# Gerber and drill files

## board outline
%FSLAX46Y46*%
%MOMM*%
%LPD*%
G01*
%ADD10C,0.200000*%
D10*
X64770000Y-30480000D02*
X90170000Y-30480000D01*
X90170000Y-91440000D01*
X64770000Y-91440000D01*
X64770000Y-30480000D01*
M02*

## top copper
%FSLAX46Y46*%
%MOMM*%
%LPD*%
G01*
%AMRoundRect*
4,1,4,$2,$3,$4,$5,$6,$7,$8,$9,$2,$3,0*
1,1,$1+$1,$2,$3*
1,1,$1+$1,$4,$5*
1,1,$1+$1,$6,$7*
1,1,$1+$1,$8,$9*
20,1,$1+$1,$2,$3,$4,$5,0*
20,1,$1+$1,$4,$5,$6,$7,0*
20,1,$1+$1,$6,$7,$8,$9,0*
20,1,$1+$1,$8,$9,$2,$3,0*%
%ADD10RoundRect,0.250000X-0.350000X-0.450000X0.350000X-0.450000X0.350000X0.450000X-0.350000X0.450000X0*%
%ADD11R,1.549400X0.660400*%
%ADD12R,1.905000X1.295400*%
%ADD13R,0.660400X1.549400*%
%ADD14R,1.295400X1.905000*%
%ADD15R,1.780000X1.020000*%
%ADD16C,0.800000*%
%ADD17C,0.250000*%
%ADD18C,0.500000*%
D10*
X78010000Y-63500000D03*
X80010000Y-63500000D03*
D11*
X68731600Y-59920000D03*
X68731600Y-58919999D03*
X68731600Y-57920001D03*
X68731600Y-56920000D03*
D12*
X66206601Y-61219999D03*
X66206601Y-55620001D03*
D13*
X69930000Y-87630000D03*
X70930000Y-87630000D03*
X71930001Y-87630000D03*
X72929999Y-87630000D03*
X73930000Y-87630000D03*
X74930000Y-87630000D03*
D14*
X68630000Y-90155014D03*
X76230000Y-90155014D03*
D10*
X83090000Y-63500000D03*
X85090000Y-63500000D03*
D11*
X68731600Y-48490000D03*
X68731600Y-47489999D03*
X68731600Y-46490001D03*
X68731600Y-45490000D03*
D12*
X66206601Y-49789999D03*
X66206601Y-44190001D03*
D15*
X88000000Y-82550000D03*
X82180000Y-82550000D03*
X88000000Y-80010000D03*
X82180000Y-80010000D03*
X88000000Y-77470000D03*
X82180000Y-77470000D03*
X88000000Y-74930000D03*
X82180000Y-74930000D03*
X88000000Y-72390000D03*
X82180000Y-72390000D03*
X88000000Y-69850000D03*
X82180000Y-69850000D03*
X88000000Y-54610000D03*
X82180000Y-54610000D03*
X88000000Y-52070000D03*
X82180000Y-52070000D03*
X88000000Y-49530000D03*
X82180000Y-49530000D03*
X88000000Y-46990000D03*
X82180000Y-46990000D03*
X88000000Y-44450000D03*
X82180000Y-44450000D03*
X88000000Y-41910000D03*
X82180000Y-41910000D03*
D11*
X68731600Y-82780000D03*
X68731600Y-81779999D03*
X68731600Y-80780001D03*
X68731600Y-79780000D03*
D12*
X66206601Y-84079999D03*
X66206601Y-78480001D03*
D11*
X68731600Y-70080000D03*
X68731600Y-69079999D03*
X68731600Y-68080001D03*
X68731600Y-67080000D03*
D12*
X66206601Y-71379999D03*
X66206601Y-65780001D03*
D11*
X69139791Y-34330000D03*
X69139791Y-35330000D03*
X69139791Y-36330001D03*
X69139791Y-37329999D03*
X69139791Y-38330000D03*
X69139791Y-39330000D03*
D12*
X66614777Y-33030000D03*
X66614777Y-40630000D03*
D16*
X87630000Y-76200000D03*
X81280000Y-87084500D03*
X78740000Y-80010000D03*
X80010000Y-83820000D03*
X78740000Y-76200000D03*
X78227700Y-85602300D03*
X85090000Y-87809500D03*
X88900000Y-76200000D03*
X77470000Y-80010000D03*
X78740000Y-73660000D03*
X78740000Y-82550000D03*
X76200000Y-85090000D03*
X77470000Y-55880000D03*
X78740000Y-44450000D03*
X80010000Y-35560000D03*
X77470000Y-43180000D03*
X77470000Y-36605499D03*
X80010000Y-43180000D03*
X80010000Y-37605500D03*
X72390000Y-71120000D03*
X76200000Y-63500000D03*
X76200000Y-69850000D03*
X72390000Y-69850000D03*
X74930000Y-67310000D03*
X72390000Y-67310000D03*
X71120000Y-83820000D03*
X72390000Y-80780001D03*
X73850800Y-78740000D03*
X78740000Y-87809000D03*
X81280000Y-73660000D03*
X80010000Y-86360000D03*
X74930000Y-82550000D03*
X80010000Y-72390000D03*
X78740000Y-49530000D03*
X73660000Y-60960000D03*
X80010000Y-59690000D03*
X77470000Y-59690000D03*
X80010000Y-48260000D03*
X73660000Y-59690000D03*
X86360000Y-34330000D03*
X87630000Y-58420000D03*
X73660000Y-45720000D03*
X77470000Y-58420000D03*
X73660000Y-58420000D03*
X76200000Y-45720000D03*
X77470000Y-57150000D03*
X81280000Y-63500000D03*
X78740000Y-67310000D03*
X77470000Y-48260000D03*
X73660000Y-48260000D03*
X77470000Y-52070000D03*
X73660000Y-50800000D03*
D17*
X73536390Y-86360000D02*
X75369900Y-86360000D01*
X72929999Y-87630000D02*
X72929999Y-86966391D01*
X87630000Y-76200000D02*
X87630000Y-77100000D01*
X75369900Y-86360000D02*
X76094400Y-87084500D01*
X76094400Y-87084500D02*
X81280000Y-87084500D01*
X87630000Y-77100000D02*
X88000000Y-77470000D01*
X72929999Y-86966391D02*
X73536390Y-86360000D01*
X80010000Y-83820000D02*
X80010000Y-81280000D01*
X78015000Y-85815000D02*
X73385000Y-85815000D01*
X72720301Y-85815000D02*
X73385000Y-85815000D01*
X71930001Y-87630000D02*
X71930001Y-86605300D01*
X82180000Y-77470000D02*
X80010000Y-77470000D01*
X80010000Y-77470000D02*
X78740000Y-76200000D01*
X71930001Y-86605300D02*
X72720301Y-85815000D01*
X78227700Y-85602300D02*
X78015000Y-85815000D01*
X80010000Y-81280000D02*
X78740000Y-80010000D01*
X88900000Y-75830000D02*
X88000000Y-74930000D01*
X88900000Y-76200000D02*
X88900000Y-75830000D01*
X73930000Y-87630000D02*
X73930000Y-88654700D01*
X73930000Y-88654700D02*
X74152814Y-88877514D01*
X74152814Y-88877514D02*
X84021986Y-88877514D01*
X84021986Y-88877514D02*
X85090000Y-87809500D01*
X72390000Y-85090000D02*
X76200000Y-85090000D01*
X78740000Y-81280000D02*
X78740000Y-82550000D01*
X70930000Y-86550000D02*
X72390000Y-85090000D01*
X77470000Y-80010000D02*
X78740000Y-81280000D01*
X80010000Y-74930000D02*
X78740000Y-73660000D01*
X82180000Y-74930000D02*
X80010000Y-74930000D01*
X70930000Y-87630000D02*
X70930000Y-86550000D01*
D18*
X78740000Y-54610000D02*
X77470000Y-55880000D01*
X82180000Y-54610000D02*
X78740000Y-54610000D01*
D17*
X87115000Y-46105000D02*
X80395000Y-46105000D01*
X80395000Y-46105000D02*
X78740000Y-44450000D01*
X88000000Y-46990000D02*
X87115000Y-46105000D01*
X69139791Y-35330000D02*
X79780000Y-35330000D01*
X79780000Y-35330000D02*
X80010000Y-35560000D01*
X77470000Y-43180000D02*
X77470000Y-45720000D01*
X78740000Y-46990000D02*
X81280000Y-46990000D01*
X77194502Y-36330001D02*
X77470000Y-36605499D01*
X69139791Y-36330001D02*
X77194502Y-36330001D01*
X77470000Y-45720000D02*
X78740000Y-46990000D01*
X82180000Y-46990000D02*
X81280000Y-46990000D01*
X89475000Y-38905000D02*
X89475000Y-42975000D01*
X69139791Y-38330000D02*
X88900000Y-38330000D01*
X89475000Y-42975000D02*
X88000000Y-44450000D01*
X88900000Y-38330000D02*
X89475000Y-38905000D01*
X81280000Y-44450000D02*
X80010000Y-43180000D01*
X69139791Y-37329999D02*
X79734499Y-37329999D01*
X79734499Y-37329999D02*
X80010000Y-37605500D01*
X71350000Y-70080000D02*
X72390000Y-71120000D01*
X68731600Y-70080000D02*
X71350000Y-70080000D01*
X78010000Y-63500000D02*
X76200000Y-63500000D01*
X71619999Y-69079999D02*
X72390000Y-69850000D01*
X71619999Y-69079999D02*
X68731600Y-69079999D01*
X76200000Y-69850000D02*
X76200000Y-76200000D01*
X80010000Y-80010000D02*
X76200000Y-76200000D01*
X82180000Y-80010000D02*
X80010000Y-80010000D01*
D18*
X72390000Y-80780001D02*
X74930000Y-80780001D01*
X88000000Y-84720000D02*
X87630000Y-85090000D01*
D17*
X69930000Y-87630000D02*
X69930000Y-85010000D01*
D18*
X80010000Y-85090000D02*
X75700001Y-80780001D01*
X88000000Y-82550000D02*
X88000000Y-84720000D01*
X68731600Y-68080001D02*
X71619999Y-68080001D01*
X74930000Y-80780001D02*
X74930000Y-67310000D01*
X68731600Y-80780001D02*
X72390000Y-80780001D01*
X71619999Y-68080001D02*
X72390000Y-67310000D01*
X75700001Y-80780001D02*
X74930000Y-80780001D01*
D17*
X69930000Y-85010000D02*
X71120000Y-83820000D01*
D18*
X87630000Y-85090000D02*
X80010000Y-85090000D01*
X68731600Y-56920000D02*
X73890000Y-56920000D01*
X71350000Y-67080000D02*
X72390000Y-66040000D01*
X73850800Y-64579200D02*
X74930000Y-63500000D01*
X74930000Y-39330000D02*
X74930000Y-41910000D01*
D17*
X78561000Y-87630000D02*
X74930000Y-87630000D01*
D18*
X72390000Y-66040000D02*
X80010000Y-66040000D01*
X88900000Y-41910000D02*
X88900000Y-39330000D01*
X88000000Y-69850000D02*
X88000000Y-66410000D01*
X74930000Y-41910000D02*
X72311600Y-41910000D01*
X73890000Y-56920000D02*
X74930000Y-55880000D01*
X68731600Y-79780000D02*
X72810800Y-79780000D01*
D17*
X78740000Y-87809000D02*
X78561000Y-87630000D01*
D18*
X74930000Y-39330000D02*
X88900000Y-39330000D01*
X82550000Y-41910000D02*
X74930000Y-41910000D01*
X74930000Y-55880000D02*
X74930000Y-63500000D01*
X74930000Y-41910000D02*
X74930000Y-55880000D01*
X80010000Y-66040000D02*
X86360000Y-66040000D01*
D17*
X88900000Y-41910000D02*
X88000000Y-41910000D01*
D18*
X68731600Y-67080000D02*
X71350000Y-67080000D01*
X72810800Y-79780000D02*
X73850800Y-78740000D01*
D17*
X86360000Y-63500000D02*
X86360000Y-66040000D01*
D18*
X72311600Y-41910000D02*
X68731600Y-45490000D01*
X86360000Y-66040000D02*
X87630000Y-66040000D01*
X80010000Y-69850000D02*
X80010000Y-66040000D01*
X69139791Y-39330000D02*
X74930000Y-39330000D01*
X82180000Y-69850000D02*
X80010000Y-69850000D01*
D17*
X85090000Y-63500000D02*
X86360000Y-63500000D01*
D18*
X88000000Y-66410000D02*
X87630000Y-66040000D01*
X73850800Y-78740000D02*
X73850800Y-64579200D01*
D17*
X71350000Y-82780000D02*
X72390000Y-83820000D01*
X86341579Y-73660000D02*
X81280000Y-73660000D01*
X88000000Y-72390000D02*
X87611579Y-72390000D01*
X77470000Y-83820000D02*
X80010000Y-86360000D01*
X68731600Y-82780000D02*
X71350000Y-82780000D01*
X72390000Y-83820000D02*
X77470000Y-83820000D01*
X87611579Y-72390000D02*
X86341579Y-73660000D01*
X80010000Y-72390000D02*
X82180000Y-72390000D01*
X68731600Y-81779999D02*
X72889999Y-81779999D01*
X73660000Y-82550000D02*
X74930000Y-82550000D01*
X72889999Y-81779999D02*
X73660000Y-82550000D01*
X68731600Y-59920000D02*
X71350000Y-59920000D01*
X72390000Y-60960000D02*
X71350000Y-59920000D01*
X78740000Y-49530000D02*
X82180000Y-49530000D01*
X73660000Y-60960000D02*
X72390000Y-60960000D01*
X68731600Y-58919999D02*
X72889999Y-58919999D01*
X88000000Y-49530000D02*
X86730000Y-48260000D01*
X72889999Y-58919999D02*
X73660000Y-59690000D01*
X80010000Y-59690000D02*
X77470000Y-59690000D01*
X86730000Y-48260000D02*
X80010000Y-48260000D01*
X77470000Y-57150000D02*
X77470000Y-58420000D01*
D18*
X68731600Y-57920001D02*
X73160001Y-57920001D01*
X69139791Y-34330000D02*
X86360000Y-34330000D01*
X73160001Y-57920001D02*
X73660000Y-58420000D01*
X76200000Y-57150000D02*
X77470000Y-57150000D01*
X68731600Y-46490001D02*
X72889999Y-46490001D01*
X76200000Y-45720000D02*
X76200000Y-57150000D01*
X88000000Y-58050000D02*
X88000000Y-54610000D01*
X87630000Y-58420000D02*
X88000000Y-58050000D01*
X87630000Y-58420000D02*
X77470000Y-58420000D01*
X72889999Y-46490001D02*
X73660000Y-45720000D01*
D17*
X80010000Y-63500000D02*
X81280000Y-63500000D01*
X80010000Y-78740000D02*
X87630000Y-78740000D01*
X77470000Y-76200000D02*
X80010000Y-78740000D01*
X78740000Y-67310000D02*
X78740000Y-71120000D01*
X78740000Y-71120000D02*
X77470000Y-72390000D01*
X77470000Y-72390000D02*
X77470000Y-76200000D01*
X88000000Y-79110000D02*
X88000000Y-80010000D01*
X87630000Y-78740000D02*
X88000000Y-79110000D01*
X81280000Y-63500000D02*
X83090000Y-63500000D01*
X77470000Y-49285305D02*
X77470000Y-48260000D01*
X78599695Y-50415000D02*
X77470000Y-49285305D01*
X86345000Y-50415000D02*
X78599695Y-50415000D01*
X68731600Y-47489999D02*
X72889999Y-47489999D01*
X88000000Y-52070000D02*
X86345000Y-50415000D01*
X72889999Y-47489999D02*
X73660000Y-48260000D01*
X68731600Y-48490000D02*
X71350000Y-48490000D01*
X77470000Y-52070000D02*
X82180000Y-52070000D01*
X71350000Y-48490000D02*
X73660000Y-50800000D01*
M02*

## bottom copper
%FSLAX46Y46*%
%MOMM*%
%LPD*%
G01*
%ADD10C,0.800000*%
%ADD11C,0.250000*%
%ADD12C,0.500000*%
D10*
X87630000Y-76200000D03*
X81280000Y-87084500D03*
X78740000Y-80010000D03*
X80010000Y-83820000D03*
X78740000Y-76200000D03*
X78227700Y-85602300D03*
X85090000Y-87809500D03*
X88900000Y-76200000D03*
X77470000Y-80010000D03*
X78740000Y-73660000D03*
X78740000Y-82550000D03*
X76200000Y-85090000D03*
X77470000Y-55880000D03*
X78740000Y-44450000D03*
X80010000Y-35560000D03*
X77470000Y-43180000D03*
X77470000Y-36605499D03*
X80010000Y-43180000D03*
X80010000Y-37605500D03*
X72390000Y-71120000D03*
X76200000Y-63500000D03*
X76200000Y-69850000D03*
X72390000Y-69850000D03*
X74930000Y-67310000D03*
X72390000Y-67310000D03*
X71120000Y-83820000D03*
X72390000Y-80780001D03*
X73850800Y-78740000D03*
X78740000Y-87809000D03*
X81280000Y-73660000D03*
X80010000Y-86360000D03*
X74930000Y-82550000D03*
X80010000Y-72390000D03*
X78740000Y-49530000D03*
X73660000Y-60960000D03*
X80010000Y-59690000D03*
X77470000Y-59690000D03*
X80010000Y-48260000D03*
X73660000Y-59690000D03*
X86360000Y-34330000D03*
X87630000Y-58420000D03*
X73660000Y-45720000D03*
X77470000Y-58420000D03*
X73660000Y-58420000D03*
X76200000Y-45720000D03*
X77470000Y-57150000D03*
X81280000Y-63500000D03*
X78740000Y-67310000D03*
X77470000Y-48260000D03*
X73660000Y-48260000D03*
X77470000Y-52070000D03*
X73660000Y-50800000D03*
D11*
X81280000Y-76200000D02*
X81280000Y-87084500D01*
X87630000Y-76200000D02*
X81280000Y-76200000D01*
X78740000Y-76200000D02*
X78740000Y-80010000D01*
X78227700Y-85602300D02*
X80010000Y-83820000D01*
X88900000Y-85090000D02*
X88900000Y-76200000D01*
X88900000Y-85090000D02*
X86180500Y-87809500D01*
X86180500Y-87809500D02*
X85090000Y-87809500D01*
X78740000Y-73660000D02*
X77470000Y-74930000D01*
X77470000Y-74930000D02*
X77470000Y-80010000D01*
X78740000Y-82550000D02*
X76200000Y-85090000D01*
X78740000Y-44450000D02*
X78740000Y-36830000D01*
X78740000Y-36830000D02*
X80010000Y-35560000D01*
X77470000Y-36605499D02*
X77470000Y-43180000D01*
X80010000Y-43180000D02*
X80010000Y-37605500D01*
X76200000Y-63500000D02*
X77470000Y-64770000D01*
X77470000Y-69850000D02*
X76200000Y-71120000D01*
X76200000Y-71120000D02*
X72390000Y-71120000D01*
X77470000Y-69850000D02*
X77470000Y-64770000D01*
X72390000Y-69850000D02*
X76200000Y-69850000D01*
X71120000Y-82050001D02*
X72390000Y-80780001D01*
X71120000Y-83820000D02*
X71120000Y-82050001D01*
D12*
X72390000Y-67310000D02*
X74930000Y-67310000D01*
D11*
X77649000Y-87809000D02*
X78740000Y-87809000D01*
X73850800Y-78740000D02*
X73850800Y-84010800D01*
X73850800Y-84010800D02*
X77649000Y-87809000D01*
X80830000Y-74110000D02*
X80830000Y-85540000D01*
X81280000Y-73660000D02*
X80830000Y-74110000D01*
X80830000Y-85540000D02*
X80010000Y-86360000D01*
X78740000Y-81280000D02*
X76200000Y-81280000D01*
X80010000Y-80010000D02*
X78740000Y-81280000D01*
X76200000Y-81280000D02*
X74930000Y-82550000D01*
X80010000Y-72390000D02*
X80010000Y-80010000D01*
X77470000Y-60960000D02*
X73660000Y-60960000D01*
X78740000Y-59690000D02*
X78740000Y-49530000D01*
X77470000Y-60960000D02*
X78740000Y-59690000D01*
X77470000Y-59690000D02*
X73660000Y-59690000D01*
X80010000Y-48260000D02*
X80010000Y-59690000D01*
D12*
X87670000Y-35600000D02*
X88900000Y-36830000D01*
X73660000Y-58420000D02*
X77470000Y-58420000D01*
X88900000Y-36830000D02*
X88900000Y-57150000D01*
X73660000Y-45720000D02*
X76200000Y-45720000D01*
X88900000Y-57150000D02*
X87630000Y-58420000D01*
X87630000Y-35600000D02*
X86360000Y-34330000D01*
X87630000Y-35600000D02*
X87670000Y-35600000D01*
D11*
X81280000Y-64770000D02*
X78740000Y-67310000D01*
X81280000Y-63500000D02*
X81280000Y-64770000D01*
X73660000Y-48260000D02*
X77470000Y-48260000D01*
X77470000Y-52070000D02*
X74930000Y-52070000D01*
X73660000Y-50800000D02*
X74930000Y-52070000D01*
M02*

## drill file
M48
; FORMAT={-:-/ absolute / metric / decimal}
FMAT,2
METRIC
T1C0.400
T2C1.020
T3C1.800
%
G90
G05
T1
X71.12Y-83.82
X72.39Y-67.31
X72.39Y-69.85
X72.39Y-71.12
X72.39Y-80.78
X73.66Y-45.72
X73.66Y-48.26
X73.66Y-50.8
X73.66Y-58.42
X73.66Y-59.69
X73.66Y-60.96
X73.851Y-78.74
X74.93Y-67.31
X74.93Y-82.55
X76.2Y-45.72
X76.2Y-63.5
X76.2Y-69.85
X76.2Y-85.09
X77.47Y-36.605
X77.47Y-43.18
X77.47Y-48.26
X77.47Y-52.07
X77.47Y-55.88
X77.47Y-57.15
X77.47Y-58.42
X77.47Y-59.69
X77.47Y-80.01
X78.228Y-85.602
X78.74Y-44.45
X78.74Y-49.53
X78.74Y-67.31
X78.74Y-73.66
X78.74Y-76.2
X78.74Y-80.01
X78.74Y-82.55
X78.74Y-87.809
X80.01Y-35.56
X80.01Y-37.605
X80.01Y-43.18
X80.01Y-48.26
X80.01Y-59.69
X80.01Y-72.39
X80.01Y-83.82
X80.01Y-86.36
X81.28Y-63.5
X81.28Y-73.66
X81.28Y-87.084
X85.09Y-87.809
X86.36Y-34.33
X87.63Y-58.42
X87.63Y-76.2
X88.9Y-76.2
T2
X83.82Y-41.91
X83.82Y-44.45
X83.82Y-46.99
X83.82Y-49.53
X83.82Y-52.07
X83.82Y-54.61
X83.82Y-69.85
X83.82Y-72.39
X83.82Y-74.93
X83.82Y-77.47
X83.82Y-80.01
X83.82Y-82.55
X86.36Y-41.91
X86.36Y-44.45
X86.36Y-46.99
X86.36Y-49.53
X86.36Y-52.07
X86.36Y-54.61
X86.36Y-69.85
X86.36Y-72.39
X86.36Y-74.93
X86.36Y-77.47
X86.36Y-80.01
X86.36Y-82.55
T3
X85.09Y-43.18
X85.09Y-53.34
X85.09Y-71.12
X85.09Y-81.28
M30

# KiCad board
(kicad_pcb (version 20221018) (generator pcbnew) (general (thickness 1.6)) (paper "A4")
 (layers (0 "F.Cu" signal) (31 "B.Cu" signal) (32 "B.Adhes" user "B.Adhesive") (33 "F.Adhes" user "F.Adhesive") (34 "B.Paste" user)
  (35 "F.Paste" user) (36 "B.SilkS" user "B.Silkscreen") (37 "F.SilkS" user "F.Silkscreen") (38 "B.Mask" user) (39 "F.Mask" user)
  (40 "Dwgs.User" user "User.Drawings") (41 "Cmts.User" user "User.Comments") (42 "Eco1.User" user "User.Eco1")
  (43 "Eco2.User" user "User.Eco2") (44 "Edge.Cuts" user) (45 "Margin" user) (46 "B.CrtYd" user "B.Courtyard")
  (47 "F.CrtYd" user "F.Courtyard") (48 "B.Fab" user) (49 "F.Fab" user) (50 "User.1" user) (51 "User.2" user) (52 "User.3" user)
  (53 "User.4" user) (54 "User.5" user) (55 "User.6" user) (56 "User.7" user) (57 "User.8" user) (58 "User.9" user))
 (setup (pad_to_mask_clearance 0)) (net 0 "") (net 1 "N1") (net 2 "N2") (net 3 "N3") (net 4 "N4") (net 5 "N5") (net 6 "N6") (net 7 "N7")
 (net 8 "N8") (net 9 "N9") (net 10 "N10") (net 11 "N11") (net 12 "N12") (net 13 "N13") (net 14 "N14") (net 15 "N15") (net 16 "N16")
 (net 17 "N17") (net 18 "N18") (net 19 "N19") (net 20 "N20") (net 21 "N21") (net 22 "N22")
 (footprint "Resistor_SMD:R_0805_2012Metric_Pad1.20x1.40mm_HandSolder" (layer "F.Cu") (at 79.01 63.5)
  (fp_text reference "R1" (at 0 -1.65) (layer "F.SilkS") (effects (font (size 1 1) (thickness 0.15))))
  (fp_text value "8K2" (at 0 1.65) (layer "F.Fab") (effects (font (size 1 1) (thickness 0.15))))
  (pad "1" smd roundrect (at -1 0) (size 1.2 1.4) (layers "F.Cu" "F.Paste" "F.Mask") (roundrect_rratio 0.2083333333) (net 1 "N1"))
  (pad "2" smd roundrect (at 1 0) (size 1.2 1.4) (layers "F.Cu" "F.Paste" "F.Mask") (roundrect_rratio 0.2083333333) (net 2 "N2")))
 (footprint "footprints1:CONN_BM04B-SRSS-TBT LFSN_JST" (layer "F.Cu") (at 67.31 58.42 90)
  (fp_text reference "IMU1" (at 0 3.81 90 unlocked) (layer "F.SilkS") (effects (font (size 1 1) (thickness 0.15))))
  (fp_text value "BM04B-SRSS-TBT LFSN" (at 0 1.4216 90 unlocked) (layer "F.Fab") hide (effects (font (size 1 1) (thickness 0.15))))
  (pad "1" smd rect (at -1.5 1.4216 90) (size 0.6604 1.5494) (layers "F.Cu" "F.Paste" "F.Mask") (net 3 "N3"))
  (pad "2" smd rect (at -0.499999 1.4216 90) (size 0.6604 1.5494) (layers "F.Cu" "F.Paste" "F.Mask") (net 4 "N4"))
  (pad "3" smd rect (at 0.499999 1.4216 90) (size 0.6604 1.5494) (layers "F.Cu" "F.Paste" "F.Mask") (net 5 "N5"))
  (pad "4" smd rect (at 1.5 1.4216 90) (size 0.6604 1.5494) (layers "F.Cu" "F.Paste" "F.Mask") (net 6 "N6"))
  (pad "5" smd rect (at -2.799999 -1.103399 180) (size 1.905 1.2954) (layers "F.Cu" "F.Paste" "F.Mask"))
  (pad "6" smd rect (at 2.799999 -1.103399 180) (size 1.905 1.2954) (layers "F.Cu" "F.Paste" "F.Mask")))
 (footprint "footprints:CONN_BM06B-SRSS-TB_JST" (layer "F.Cu") (at 72.43 89.459791)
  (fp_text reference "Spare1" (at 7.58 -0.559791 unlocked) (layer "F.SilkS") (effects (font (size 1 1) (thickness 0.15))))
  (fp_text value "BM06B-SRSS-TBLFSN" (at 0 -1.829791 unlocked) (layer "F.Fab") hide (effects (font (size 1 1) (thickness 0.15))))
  (pad "1" smd rect (at -2.5 -1.829791) (size 0.6604 1.5494) (layers "F.Cu" "F.Paste" "F.Mask") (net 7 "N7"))
  (pad "2" smd rect (at -1.5 -1.829791) (size 0.6604 1.5494) (layers "F.Cu" "F.Paste" "F.Mask") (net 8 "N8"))
  (pad "3" smd rect (at -0.499999 -1.829791) (size 0.6604 1.5494) (layers "F.Cu" "F.Paste" "F.Mask") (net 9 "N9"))
  (pad "4" smd rect (at 0.499999 -1.829791) (size 0.6604 1.5494) (layers "F.Cu" "F.Paste" "F.Mask") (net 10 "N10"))
  (pad "5" smd rect (at 1.5 -1.829791) (size 0.6604 1.5494) (layers "F.Cu" "F.Paste" "F.Mask") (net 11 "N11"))
  (pad "6" smd rect (at 2.5 -1.829791) (size 0.6604 1.5494) (layers "F.Cu" "F.Paste" "F.Mask") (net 6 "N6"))
  (pad "7" smd rect (at -3.8 0.695223 90) (size 1.905 1.2954) (layers "F.Cu" "F.Paste" "F.Mask"))
  (pad "8" smd rect (at 3.8 0.695223 90) (size 1.905 1.2954) (layers "F.Cu" "F.Paste" "F.Mask")))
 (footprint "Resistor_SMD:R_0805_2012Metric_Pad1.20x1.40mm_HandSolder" (layer "F.Cu") (at 84.09 63.5)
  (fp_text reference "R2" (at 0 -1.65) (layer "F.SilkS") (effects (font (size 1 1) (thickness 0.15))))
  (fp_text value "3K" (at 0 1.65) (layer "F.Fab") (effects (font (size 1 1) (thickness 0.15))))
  (pad "1" smd roundrect (at -1 0) (size 1.2 1.4) (layers "F.Cu" "F.Paste" "F.Mask") (roundrect_rratio 0.2083333333) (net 2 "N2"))
  (pad "2" smd roundrect (at 1 0) (size 1.2 1.4) (layers "F.Cu" "F.Paste" "F.Mask") (roundrect_rratio 0.2083333333) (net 6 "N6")))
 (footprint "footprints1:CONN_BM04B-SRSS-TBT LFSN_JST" (layer "F.Cu") (at 67.31 46.99 90)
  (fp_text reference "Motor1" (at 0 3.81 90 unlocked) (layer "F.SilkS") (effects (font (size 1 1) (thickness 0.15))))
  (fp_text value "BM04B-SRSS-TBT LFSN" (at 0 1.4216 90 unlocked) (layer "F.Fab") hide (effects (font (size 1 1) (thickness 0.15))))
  (pad "1" smd rect (at -1.5 1.4216 90) (size 0.6604 1.5494) (layers "F.Cu" "F.Paste" "F.Mask") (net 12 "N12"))
  (pad "2" smd rect (at -0.499999 1.4216 90) (size 0.6604 1.5494) (layers "F.Cu" "F.Paste" "F.Mask") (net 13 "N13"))
  (pad "3" smd rect (at 0.499999 1.4216 90) (size 0.6604 1.5494) (layers "F.Cu" "F.Paste" "F.Mask") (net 5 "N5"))
  (pad "4" smd rect (at 1.5 1.4216 90) (size 0.6604 1.5494) (layers "F.Cu" "F.Paste" "F.Mask") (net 6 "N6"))
  (pad "5" smd rect (at -2.799999 -1.103399 180) (size 1.905 1.2954) (layers "F.Cu" "F.Paste" "F.Mask"))
  (pad "6" smd rect (at 2.799999 -1.103399 180) (size 1.905 1.2954) (layers "F.Cu" "F.Paste" "F.Mask")))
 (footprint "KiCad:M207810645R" (layer "F.Cu") (at 85.09 76.2 90)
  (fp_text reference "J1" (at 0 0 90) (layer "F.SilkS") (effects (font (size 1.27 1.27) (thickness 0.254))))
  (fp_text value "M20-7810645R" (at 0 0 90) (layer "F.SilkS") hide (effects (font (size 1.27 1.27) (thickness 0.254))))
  (pad "" np_thru_hole circle (at -6.35 -1.27 90) (size 1.02 1.02) (drill 1.02) (layers "*.Cu" "*.Mask"))
  (pad "" np_thru_hole circle (at -6.35 1.27 90) (size 1.02 1.02) (drill 1.02) (layers "*.Cu" "*.Mask"))
  (pad "" np_thru_hole circle (at -5.08 0 90) (size 1.8 1.8) (drill 1.8) (layers "*.Cu" "*.Mask"))
  (pad "" np_thru_hole circle (at -3.81 -1.27 90) (size 1.02 1.02) (drill 1.02) (layers "*.Cu" "*.Mask"))
  (pad "" np_thru_hole circle (at -3.81 1.27 90) (size 1.02 1.02) (drill 1.02) (layers "*.Cu" "*.Mask"))
  (pad "" np_thru_hole circle (at -1.27 -1.27 90) (size 1.02 1.02) (drill 1.02) (layers "*.Cu" "*.Mask"))
  (pad "" np_thru_hole circle (at -1.27 1.27 90) (size 1.02 1.02) (drill 1.02) (layers "*.Cu" "*.Mask"))
  (pad "" np_thru_hole circle (at 1.27 -1.27 90) (size 1.02 1.02) (drill 1.02) (layers "*.Cu" "*.Mask"))
  (pad "" np_thru_hole circle (at 1.27 1.27 90) (size 1.02 1.02) (drill 1.02) (layers "*.Cu" "*.Mask"))
  (pad "" np_thru_hole circle (at 3.81 -1.27 90) (size 1.02 1.02) (drill 1.02) (layers "*.Cu" "*.Mask"))
  (pad "" np_thru_hole circle (at 3.81 1.27 90) (size 1.02 1.02) (drill 1.02) (layers "*.Cu" "*.Mask"))
  (pad "" np_thru_hole circle (at 5.08 0 90) (size 1.8 1.8) (drill 1.8) (layers "*.Cu" "*.Mask"))
  (pad "" np_thru_hole circle (at 6.35 -1.27 90) (size 1.02 1.02) (drill 1.02) (layers "*.Cu" "*.Mask"))
  (pad "" np_thru_hole circle (at 6.35 1.27 90) (size 1.02 1.02) (drill 1.02) (layers "*.Cu" "*.Mask"))
  (pad "1" smd rect (at -6.35 2.91 90) (size 1.02 1.78) (layers "F.Cu" "F.Paste" "F.Mask") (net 7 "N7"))
  (pad "2" smd rect (at -6.35 -2.91 90) (size 1.02 1.78) (layers "F.Cu" "F.Paste" "F.Mask") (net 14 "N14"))
  (pad "3" smd rect (at -3.81 2.91 90) (size 1.02 1.78) (layers "F.Cu" "F.Paste" "F.Mask") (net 2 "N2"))
  (pad "4" smd rect (at -3.81 -2.91 90) (size 1.02 1.78) (layers "F.Cu" "F.Paste" "F.Mask") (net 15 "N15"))
  (pad "5" smd rect (at -1.27 2.91 90) (size 1.02 1.78) (layers "F.Cu" "F.Paste" "F.Mask") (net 10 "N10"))
  (pad "6" smd rect (at -1.27 -2.91 90) (size 1.02 1.78) (layers "F.Cu" "F.Paste" "F.Mask") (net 9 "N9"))
  (pad "7" smd rect (at 1.27 2.91 90) (size 1.02 1.78) (layers "F.Cu" "F.Paste" "F.Mask") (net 11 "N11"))
  (pad "8" smd rect (at 1.27 -2.91 90) (size 1.02 1.78) (layers "F.Cu" "F.Paste" "F.Mask") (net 8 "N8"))
  (pad "9" smd rect (at 3.81 2.91 90) (size 1.02 1.78) (layers "F.Cu" "F.Paste" "F.Mask") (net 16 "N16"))
  (pad "10" smd rect (at 3.81 -2.91 90) (size 1.02 1.78) (layers "F.Cu" "F.Paste" "F.Mask") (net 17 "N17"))
  (pad "11" smd rect (at 6.35 2.91 90) (size 1.02 1.78) (layers "F.Cu" "F.Paste" "F.Mask") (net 6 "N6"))
  (pad "12" smd rect (at 6.35 -2.91 90) (size 1.02 1.78) (layers "F.Cu" "F.Paste" "F.Mask") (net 6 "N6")))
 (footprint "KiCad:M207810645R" (layer "F.Cu") (at 85.09 48.26 90)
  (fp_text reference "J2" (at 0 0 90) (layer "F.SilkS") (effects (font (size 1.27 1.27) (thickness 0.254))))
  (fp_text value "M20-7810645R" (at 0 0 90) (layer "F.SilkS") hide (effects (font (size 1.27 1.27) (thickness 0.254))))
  (pad "" np_thru_hole circle (at -6.35 -1.27 90) (size 1.02 1.02) (drill 1.02) (layers "*.Cu" "*.Mask"))
  (pad "" np_thru_hole circle (at -6.35 1.27 90) (size 1.02 1.02) (drill 1.02) (layers "*.Cu" "*.Mask"))
  (pad "" np_thru_hole circle (at -5.08 0 90) (size 1.8 1.8) (drill 1.8) (layers "*.Cu" "*.Mask"))
  (pad "" np_thru_hole circle (at -3.81 -1.27 90) (size 1.02 1.02) (drill 1.02) (layers "*.Cu" "*.Mask"))
  (pad "" np_thru_hole circle (at -3.81 1.27 90) (size 1.02 1.02) (drill 1.02) (layers "*.Cu" "*.Mask"))
  (pad "" np_thru_hole circle (at -1.27 -1.27 90) (size 1.02 1.02) (drill 1.02) (layers "*.Cu" "*.Mask"))
  (pad "" np_thru_hole circle (at -1.27 1.27 90) (size 1.02 1.02) (drill 1.02) (layers "*.Cu" "*.Mask"))
  (pad "" np_thru_hole circle (at 1.27 -1.27 90) (size 1.02 1.02) (drill 1.02) (layers "*.Cu" "*.Mask"))
  (pad "" np_thru_hole circle (at 1.27 1.27 90) (size 1.02 1.02) (drill 1.02) (layers "*.Cu" "*.Mask"))
  (pad "" np_thru_hole circle (at 3.81 -1.27 90) (size 1.02 1.02) (drill 1.02) (layers "*.Cu" "*.Mask"))
  (pad "" np_thru_hole circle (at 3.81 1.27 90) (size 1.02 1.02) (drill 1.02) (layers "*.Cu" "*.Mask"))
  (pad "" np_thru_hole circle (at 5.08 0 90) (size 1.8 1.8) (drill 1.8) (layers "*.Cu" "*.Mask"))
  (pad "" np_thru_hole circle (at 6.35 -1.27 90) (size 1.02 1.02) (drill 1.02) (layers "*.Cu" "*.Mask"))
  (pad "" np_thru_hole circle (at 6.35 1.27 90) (size 1.02 1.02) (drill 1.02) (layers "*.Cu" "*.Mask"))
  (pad "1" smd rect (at -6.35 2.91 90) (size 1.02 1.78) (layers "F.Cu" "F.Paste" "F.Mask") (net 5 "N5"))
  (pad "2" smd rect (at -6.35 -2.91 90) (size 1.02 1.78) (layers "F.Cu" "F.Paste" "F.Mask") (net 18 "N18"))
  (pad "3" smd rect (at -3.81 2.91 90) (size 1.02 1.78) (layers "F.Cu" "F.Paste" "F.Mask") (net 13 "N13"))
  (pad "4" smd rect (at -3.81 -2.91 90) (size 1.02 1.78) (layers "F.Cu" "F.Paste" "F.Mask") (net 12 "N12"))
  (pad "5" smd rect (at -1.27 2.91 90) (size 1.02 1.78) (layers "F.Cu" "F.Paste" "F.Mask") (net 4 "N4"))
  (pad "6" smd rect (at -1.27 -2.91 90) (size 1.02 1.78) (layers "F.Cu" "F.Paste" "F.Mask") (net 3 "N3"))
  (pad "7" smd rect (at 1.27 2.91 90) (size 1.02 1.78) (layers "F.Cu" "F.Paste" "F.Mask") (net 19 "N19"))
  (pad "8" smd rect (at 1.27 -2.91 90) (size 1.02 1.78) (layers "F.Cu" "F.Paste" "F.Mask") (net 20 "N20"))
  (pad "9" smd rect (at 3.81 2.91 90) (size 1.02 1.78) (layers "F.Cu" "F.Paste" "F.Mask") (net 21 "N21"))
  (pad "10" smd rect (at 3.81 -2.91 90) (size 1.02 1.78) (layers "F.Cu" "F.Paste" "F.Mask") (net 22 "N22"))
  (pad "11" smd rect (at 6.35 2.91 90) (size 1.02 1.78) (layers "F.Cu" "F.Paste" "F.Mask") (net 6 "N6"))
  (pad "12" smd rect (at 6.35 -2.91 90) (size 1.02 1.78) (layers "F.Cu" "F.Paste" "F.Mask") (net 6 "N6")))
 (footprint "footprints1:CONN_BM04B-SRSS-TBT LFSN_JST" (layer "F.Cu") (at 67.31 81.28 90)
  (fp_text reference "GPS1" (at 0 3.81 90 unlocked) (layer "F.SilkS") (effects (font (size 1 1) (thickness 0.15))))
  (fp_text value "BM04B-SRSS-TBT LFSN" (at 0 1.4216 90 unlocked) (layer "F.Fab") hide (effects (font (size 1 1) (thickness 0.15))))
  (pad "1" smd rect (at -1.5 1.4216 90) (size 0.6604 1.5494) (layers "F.Cu" "F.Paste" "F.Mask") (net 16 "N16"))
  (pad "2" smd rect (at -0.499999 1.4216 90) (size 0.6604 1.5494) (layers "F.Cu" "F.Paste" "F.Mask") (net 17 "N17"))
  (pad "3" smd rect (at 0.499999 1.4216 90) (size 0.6604 1.5494) (layers "F.Cu" "F.Paste" "F.Mask") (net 7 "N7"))
  (pad "4" smd rect (at 1.5 1.4216 90) (size 0.6604 1.5494) (layers "F.Cu" "F.Paste" "F.Mask") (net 6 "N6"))
  (pad "5" smd rect (at -2.799999 -1.103399 180) (size 1.905 1.2954) (layers "F.Cu" "F.Paste" "F.Mask"))
  (pad "6" smd rect (at 2.799999 -1.103399 180) (size 1.905 1.2954) (layers "F.Cu" "F.Paste" "F.Mask")))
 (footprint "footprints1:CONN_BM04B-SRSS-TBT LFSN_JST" (layer "F.Cu") (at 67.31 68.58 90)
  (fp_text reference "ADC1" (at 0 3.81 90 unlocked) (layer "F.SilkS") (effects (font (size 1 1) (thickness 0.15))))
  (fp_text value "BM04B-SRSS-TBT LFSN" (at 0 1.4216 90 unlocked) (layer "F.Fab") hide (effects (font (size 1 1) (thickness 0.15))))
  (pad "1" smd rect (at -1.5 1.4216 90) (size 0.6604 1.5494) (layers "F.Cu" "F.Paste" "F.Mask") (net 1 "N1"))
  (pad "2" smd rect (at -0.499999 1.4216 90) (size 0.6604 1.5494) (layers "F.Cu" "F.Paste" "F.Mask") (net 15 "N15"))
  (pad "3" smd rect (at 0.499999 1.4216 90) (size 0.6604 1.5494) (layers "F.Cu" "F.Paste" "F.Mask") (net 7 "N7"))
  (pad "4" smd rect (at 1.5 1.4216 90) (size 0.6604 1.5494) (layers "F.Cu" "F.Paste" "F.Mask") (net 6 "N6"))
  (pad "5" smd rect (at -2.799999 -1.103399 180) (size 1.905 1.2954) (layers "F.Cu" "F.Paste" "F.Mask"))
  (pad "6" smd rect (at 2.799999 -1.103399 180) (size 1.905 1.2954) (layers "F.Cu" "F.Paste" "F.Mask")))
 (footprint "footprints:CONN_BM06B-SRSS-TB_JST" (layer "F.Cu") (at 67.31 36.83 -90)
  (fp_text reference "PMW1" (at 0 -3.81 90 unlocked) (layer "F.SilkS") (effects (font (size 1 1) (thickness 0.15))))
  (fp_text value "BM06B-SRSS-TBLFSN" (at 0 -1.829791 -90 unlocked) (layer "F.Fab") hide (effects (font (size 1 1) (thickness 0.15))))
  (pad "1" smd rect (at -2.5 -1.829791 270) (size 0.6604 1.5494) (layers "F.Cu" "F.Paste" "F.Mask") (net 5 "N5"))
  (pad "2" smd rect (at -1.5 -1.829791 270) (size 0.6604 1.5494) (layers "F.Cu" "F.Paste" "F.Mask") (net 19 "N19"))
  (pad "3" smd rect (at -0.499999 -1.829791 270) (size 0.6604 1.5494) (layers "F.Cu" "F.Paste" "F.Mask") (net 20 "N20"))
  (pad "4" smd rect (at 0.499999 -1.829791 270) (size 0.6604 1.5494) (layers "F.Cu" "F.Paste" "F.Mask") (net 22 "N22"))
  (pad "5" smd rect (at 1.5 -1.829791 270) (size 0.6604 1.5494) (layers "F.Cu" "F.Paste" "F.Mask") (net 21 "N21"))
  (pad "6" smd rect (at 2.5 -1.829791 270) (size 0.6604 1.5494) (layers "F.Cu" "F.Paste" "F.Mask") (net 6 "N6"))
  (pad "7" smd rect (at -3.8 0.695223) (size 1.905 1.2954) (layers "F.Cu" "F.Paste" "F.Mask"))
  (pad "8" smd rect (at 3.8 0.695223) (size 1.905 1.2954) (layers "F.Cu" "F.Paste" "F.Mask")))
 (gr_rect (start 64.77 30.48) (end 90.17 91.44) (stroke (width 0.2) (type default)) (fill none) (layer "Edge.Cuts"))
 (segment (start 73.53639 86.36) (end 75.3699 86.36) (width 0.25) (layer "F.Cu") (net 10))
 (segment (start 72.929999 87.63) (end 72.929999 86.966391) (width 0.25) (layer "F.Cu") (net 10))
 (segment (start 87.63 76.2) (end 87.63 77.1) (width 0.25) (layer "F.Cu") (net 10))
 (segment (start 75.3699 86.36) (end 76.0944 87.0845) (width 0.25) (layer "F.Cu") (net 10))
 (segment (start 76.0944 87.0845) (end 81.28 87.0845) (width 0.25) (layer "F.Cu") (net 10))
 (segment (start 87.63 77.1) (end 88 77.47) (width 0.25) (layer "F.Cu") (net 10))
 (segment (start 72.929999 86.966391) (end 73.53639 86.36) (width 0.25) (layer "F.Cu") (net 10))
 (via (at 87.63 76.2) (size 0.8) (drill 0.4) (layers "F.Cu" "B.Cu") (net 10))
 (via (at 81.28 87.0845) (size 0.8) (drill 0.4) (layers "F.Cu" "B.Cu") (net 10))
 (segment (start 81.28 76.2) (end 81.28 87.0845) (width 0.25) (layer "B.Cu") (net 10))
 (segment (start 87.63 76.2) (end 81.28 76.2) (width 0.25) (layer "B.Cu") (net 10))
 (segment (start 80.01 83.82) (end 80.01 81.28) (width 0.25) (layer "F.Cu") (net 9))
 (segment (start 78.015 85.815) (end 73.385 85.815) (width 0.25) (layer "F.Cu") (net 9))
 (segment (start 72.720301 85.815) (end 73.385 85.815) (width 0.25) (layer "F.Cu") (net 9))
 (segment (start 71.930001 87.63) (end 71.930001 86.6053) (width 0.25) (layer "F.Cu") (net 9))
 (segment (start 82.18 77.47) (end 80.01 77.47) (width 0.25) (layer "F.Cu") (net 9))
 (segment (start 80.01 77.47) (end 78.74 76.2) (width 0.25) (layer "F.Cu") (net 9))
 (segment (start 71.930001 86.6053) (end 72.720301 85.815) (width 0.25) (layer "F.Cu") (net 9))
 (segment (start 78.2277 85.6023) (end 78.015 85.815) (width 0.25) (layer "F.Cu") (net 9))
 (segment (start 80.01 81.28) (end 78.74 80.01) (width 0.25) (layer "F.Cu") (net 9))
 (via (at 78.74 80.01) (size 0.8) (drill 0.4) (layers "F.Cu" "B.Cu") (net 9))
 (via (at 80.01 83.82) (size 0.8) (drill 0.4) (layers "F.Cu" "B.Cu") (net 9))
 (via (at 78.74 76.2) (size 0.8) (drill 0.4) (layers "F.Cu" "B.Cu") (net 9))
 (via (at 78.2277 85.6023) (size 0.8) (drill 0.4) (layers "F.Cu" "B.Cu") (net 9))
 (segment (start 78.74 76.2) (end 78.74 80.01) (width 0.25) (layer "B.Cu") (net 9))
 (segment (start 78.2277 85.6023) (end 80.01 83.82) (width 0.25) (layer "B.Cu") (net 9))
 (segment (start 88.9 75.83) (end 88 74.93) (width 0.25) (layer "F.Cu") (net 11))
 (segment (start 88.9 76.2) (end 88.9 75.83) (width 0.25) (layer "F.Cu") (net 11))
 (segment (start 73.93 87.63) (end 73.93 88.6547) (width 0.25) (layer "F.Cu") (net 11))
 (segment (start 73.93 88.6547) (end 74.152814 88.877514) (width 0.25) (layer "F.Cu") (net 11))
 (segment (start 74.152814 88.877514) (end 84.021986 88.877514) (width 0.25) (layer "F.Cu") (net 11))
 (segment (start 84.021986 88.877514) (end 85.09 87.8095) (width 0.25) (layer "F.Cu") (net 11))
 (via (at 85.09 87.8095) (size 0.8) (drill 0.4) (layers "F.Cu" "B.Cu") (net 11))
 (via (at 88.9 76.2) (size 0.8) (drill 0.4) (layers "F.Cu" "B.Cu") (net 11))
 (segment (start 88.9 85.09) (end 88.9 76.2) (width 0.25) (layer "B.Cu") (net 11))
 (segment (start 88.9 85.09) (end 86.1805 87.8095) (width 0.25) (layer "B.Cu") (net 11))
 (segment (start 86.1805 87.8095) (end 85.09 87.8095) (width 0.25) (layer "B.Cu") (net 11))
 (segment (start 72.39 85.09) (end 76.2 85.09) (width 0.25) (layer "F.Cu") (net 8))
 (segment (start 78.74 81.28) (end 78.74 82.55) (width 0.25) (layer "F.Cu") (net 8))
 (segment (start 70.93 86.55) (end 72.39 85.09) (width 0.25) (layer "F.Cu") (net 8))
 (segment (start 77.47 80.01) (end 78.74 81.28) (width 0.25) (layer "F.Cu") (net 8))
 (segment (start 80.01 74.93) (end 78.74 73.66) (width 0.25) (layer "F.Cu") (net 8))
 (segment (start 82.18 74.93) (end 80.01 74.93) (width 0.25) (layer "F.Cu") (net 8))
 (segment (start 70.93 87.63) (end 70.93 86.55) (width 0.25) (layer "F.Cu") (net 8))
 (via (at 77.47 80.01) (size 0.8) (drill 0.4) (layers "F.Cu" "B.Cu") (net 8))
 (via (at 78.74 73.66) (size 0.8) (drill 0.4) (layers "F.Cu" "B.Cu") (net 8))
 (via (at 78.74 82.55) (size 0.8) (drill 0.4) (layers "F.Cu" "B.Cu") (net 8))
 (via (at 76.2 85.09) (size 0.8) (drill 0.4) (layers "F.Cu" "B.Cu") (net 8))
 (segment (start 78.74 73.66) (end 77.47 74.93) (width 0.25) (layer "B.Cu") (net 8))
 (segment (start 77.47 74.93) (end 77.47 80.01) (width 0.25) (layer "B.Cu") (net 8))
 (segment (start 78.74 82.55) (end 76.2 85.09) (width 0.25) (layer "B.Cu") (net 8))
 (segment (start 78.74 54.61) (end 77.47 55.88) (width 0.5) (layer "F.Cu") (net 18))
 (segment (start 82.18 54.61) (end 78.74 54.61) (width 0.5) (layer "F.Cu") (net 18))
 (via (at 77.47 55.88) (size 0.8) (drill 0.4) (layers "F.Cu" "B.Cu") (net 18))
 (segment (start 87.115 46.105) (end 80.395 46.105) (width 0.25) (layer "F.Cu") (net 19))
 (segment (start 80.395 46.105) (end 78.74 44.45) (width 0.25) (layer "F.Cu") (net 19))
 (segment (start 88 46.99) (end 87.115 46.105) (width 0.25) (layer "F.Cu") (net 19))
 (segment (start 69.139791 35.33) (end 79.78 35.33) (width 0.25) (layer "F.Cu") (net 19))
 (segment (start 79.78 35.33) (end 80.01 35.56) (width 0.25) (layer "F.Cu") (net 19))
 (via (at 78.74 44.45) (size 0.8) (drill 0.4) (layers "F.Cu" "B.Cu") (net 19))
 (via (at 80.01 35.56) (size 0.8) (drill 0.4) (layers "F.Cu" "B.Cu") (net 19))
 (segment (start 78.74 44.45) (end 78.74 36.83) (width 0.25) (layer "B.Cu") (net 19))
 (segment (start 78.74 36.83) (end 80.01 35.56) (width 0.25) (layer "B.Cu") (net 19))
 (segment (start 77.47 43.18) (end 77.47 45.72) (width 0.25) (layer "F.Cu") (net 20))
 (segment (start 78.74 46.99) (end 81.28 46.99) (width 0.25) (layer "F.Cu") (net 20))
 (segment (start 77.194502 36.330001) (end 77.47 36.605499) (width 0.25) (layer "F.Cu") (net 20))
 (segment (start 69.139791 36.330001) (end 77.194502 36.330001) (width 0.25) (layer "F.Cu") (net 20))
 (segment (start 77.47 45.72) (end 78.74 46.99) (width 0.25) (layer "F.Cu") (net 20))
 (segment (start 82.18 46.99) (end 81.28 46.99) (width 0.25) (layer "F.Cu") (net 20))
 (via (at 77.47 43.18) (size 0.8) (drill 0.4) (layers "F.Cu" "B.Cu") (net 20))
 (via (at 77.47 36.605499) (size 0.8) (drill 0.4) (layers "F.Cu" "B.Cu") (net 20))
 (segment (start 77.47 36.605499) (end 77.47 43.18) (width 0.25) (layer "B.Cu") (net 20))
 (segment (start 89.475 38.905) (end 89.475 42.975) (width 0.25) (layer "F.Cu") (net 21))
 (segment (start 69.139791 38.33) (end 88.9 38.33) (width 0.25) (layer "F.Cu") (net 21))
 (segment (start 89.475 42.975) (end 88 44.45) (width 0.25) (layer "F.Cu") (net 21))
 (segment (start 88.9 38.33) (end 89.475 38.905) (width 0.25) (layer "F.Cu") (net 21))
 (segment (start 81.28 44.45) (end 80.01 43.18) (width 0.25) (layer "F.Cu") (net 22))
 (segment (start 69.139791 37.329999) (end 79.734499 37.329999) (width 0.25) (layer "F.Cu") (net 22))
 (segment (start 79.734499 37.329999) (end 80.01 37.6055) (width 0.25) (layer "F.Cu") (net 22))
 (via (at 80.01 43.18) (size 0.8) (drill 0.4) (layers "F.Cu" "B.Cu") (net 22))
 (via (at 80.01 37.6055) (size 0.8) (drill 0.4) (layers "F.Cu" "B.Cu") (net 22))
 (segment (start 80.01 43.18) (end 80.01 37.6055) (width 0.25) (layer "B.Cu") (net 22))
 (segment (start 71.35 70.08) (end 72.39 71.12) (width 0.25) (layer "F.Cu") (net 1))
 (segment (start 68.7316 70.08) (end 71.35 70.08) (width 0.25) (layer "F.Cu") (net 1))
 (segment (start 78.01 63.5) (end 76.2 63.5) (width 0.25) (layer "F.Cu") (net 1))
 (via (at 72.39 71.12) (size 0.8) (drill 0.4) (layers "F.Cu" "B.Cu") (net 1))
 (via (at 76.2 63.5) (size 0.8) (drill 0.4) (layers "F.Cu" "B.Cu") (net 1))
 (segment (start 76.2 63.5) (end 77.47 64.77) (width 0.25) (layer "B.Cu") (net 1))
 (segment (start 77.47 69.85) (end 76.2 71.12) (width 0.25) (layer "B.Cu") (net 1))
 (segment (start 76.2 71.12) (end 72.39 71.12) (width 0.25) (layer "B.Cu") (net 1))
 (segment (start 77.47 69.85) (end 77.47 64.77) (width 0.25) (layer "B.Cu") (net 1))
 (segment (start 71.619999 69.079999) (end 72.39 69.85) (width 0.25) (layer "F.Cu") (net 15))
 (segment (start 71.619999 69.079999) (end 68.7316 69.079999) (width 0.25) (layer "F.Cu") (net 15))
 (segment (start 76.2 69.85) (end 76.2 76.2) (width 0.25) (layer "F.Cu") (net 15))
 (segment (start 80.01 80.01) (end 76.2 76.2) (width 0.25) (layer "F.Cu") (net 15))
 (segment (start 82.18 80.01) (end 80.01 80.01) (width 0.25) (layer "F.Cu") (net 15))
 (via (at 76.2 69.85) (size 0.8) (drill 0.4) (layers "F.Cu" "B.Cu") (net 15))
 (via (at 72.39 69.85) (size 0.8) (drill 0.4) (layers "F.Cu" "B.Cu") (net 15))
 (segment (start 72.39 69.85) (end 76.2 69.85) (width 0.25) (layer "B.Cu") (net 15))
 (segment (start 72.39 80.780001) (end 74.93 80.780001) (width 0.5) (layer "F.Cu") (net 7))
 (segment (start 88 84.72) (end 87.63 85.09) (width 0.5) (layer "F.Cu") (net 7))
 (segment (start 69.93 87.63) (end 69.93 85.01) (width 0.25) (layer "F.Cu") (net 7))
 (segment (start 80.01 85.09) (end 75.700001 80.780001) (width 0.5) (layer "F.Cu") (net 7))
 (segment (start 88 82.55) (end 88 84.72) (width 0.5) (layer "F.Cu") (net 7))
 (segment (start 68.7316 68.080001) (end 71.619999 68.080001) (width 0.5) (layer "F.Cu") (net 7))
 (segment (start 74.93 80.780001) (end 74.93 67.31) (width 0.5) (layer "F.Cu") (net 7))
 (segment (start 68.7316 80.780001) (end 72.39 80.780001) (width 0.5) (layer "F.Cu") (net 7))
 (segment (start 71.619999 68.080001) (end 72.39 67.31) (width 0.5) (layer "F.Cu") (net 7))
 (segment (start 75.700001 80.780001) (end 74.93 80.780001) (width 0.5) (layer "F.Cu") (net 7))
 (segment (start 69.93 85.01) (end 71.12 83.82) (width 0.25) (layer "F.Cu") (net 7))
 (segment (start 87.63 85.09) (end 80.01 85.09) (width 0.5) (layer "F.Cu") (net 7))
 (via (at 74.93 67.31) (size 0.8) (drill 0.4) (layers "F.Cu" "B.Cu") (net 7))
 (via (at 72.39 67.31) (size 0.8) (drill 0.4) (layers "F.Cu" "B.Cu") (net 7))
 (via (at 71.12 83.82) (size 0.8) (drill 0.4) (layers "F.Cu" "B.Cu") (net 7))
 (via (at 72.39 80.780001) (size 0.8) (drill 0.4) (layers "F.Cu" "B.Cu") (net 7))
 (segment (start 71.12 82.050001) (end 72.39 80.780001) (width 0.25) (layer "B.Cu") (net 7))
 (segment (start 71.12 83.82) (end 71.12 82.050001) (width 0.25) (layer "B.Cu") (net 7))
 (segment (start 72.39 67.31) (end 74.93 67.31) (width 0.5) (layer "B.Cu") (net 7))
 (segment (start 68.7316 56.92) (end 73.89 56.92) (width 0.5) (layer "F.Cu") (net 6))
 (segment (start 71.35 67.08) (end 72.39 66.04) (width 0.5) (layer "F.Cu") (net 6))
 (segment (start 73.8508 64.5792) (end 74.93 63.5) (width 0.5) (layer "F.Cu") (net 6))
 (segment (start 74.93 39.33) (end 74.93 41.91) (width 0.5) (layer "F.Cu") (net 6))
 (segment (start 78.561 87.63) (end 74.93 87.63) (width 0.25) (layer "F.Cu") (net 6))
 (segment (start 72.39 66.04) (end 80.01 66.04) (width 0.5) (layer "F.Cu") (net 6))
 (segment (start 88.9 41.91) (end 88.9 39.33) (width 0.5) (layer "F.Cu") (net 6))
 (segment (start 88 69.85) (end 88 66.41) (width 0.5) (layer "F.Cu") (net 6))
 (segment (start 74.93 41.91) (end 72.3116 41.91) (width 0.5) (layer "F.Cu") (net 6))
 (segment (start 73.89 56.92) (end 74.93 55.88) (width 0.5) (layer "F.Cu") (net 6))
 (segment (start 68.7316 79.78) (end 72.8108 79.78) (width 0.5) (layer "F.Cu") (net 6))
 (segment (start 78.74 87.809) (end 78.561 87.63) (width 0.25) (layer "F.Cu") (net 6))
 (segment (start 74.93 39.33) (end 88.9 39.33) (width 0.5) (layer "F.Cu") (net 6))
 (segment (start 82.55 41.91) (end 74.93 41.91) (width 0.5) (layer "F.Cu") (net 6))
 (segment (start 74.93 55.88) (end 74.93 63.5) (width 0.5) (layer "F.Cu") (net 6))
 (segment (start 74.93 41.91) (end 74.93 55.88) (width 0.5) (layer "F.Cu") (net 6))
 (segment (start 80.01 66.04) (end 86.36 66.04) (width 0.5) (layer "F.Cu") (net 6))
 (segment (start 88.9 41.91) (end 88 41.91) (width 0.25) (layer "F.Cu") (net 6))
 (segment (start 68.7316 67.08) (end 71.35 67.08) (width 0.5) (layer "F.Cu") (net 6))
 (segment (start 72.8108 79.78) (end 73.8508 78.74) (width 0.5) (layer "F.Cu") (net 6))
 (segment (start 86.36 63.5) (end 86.36 66.04) (width 0.25) (layer "F.Cu") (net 6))
 (segment (start 72.3116 41.91) (end 68.7316 45.49) (width 0.5) (layer "F.Cu") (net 6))
 (segment (start 86.36 66.04) (end 87.63 66.04) (width 0.5) (layer "F.Cu") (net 6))
 (segment (start 80.01 69.85) (end 80.01 66.04) (width 0.5) (layer "F.Cu") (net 6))
 (segment (start 69.139791 39.33) (end 74.93 39.33) (width 0.5) (layer "F.Cu") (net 6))
 (segment (start 82.18 69.85) (end 80.01 69.85) (width 0.5) (layer "F.Cu") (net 6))
 (segment (start 85.09 63.5) (end 86.36 63.5) (width 0.25) (layer "F.Cu") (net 6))
 (segment (start 88 66.41) (end 87.63 66.04) (width 0.5) (layer "F.Cu") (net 6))
 (segment (start 73.8508 78.74) (end 73.8508 64.5792) (width 0.5) (layer "F.Cu") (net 6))
 (via (at 73.8508 78.74) (size 0.8) (drill 0.4) (layers "F.Cu" "B.Cu") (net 6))
 (via (at 78.74 87.809) (size 0.8) (drill 0.4) (layers "F.Cu" "B.Cu") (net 6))
 (segment (start 77.649 87.809) (end 78.74 87.809) (width 0.25) (layer "B.Cu") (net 6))
 (segment (start 73.8508 78.74) (end 73.8508 84.0108) (width 0.25) (layer "B.Cu") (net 6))
 (segment (start 73.8508 84.0108) (end 77.649 87.809) (width 0.25) (layer "B.Cu") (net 6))
 (segment (start 71.35 82.78) (end 72.39 83.82) (width 0.25) (layer "F.Cu") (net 16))
 (segment (start 86.341579 73.66) (end 81.28 73.66) (width 0.25) (layer "F.Cu") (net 16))
 (segment (start 88 72.39) (end 87.611579 72.39) (width 0.25) (layer "F.Cu") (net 16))
 (segment (start 77.47 83.82) (end 80.01 86.36) (width 0.25) (layer "F.Cu") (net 16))
 (segment (start 68.7316 82.78) (end 71.35 82.78) (width 0.25) (layer "F.Cu") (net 16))
 (segment (start 72.39 83.82) (end 77.47 83.82) (width 0.25) (layer "F.Cu") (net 16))
 (segment (start 87.611579 72.39) (end 86.341579 73.66) (width 0.25) (layer "F.Cu") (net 16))
 (via (at 81.28 73.66) (size 0.8) (drill 0.4) (layers "F.Cu" "B.Cu") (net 16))
 (via (at 80.01 86.36) (size 0.8) (drill 0.4) (layers "F.Cu" "B.Cu") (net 16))
 (segment (start 80.83 74.11) (end 80.83 85.54) (width 0.25) (layer "B.Cu") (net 16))
 (segment (start 81.28 73.66) (end 80.83 74.11) (width 0.25) (layer "B.Cu") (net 16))
 (segment (start 80.83 85.54) (end 80.01 86.36) (width 0.25) (layer "B.Cu") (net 16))
 (segment (start 80.01 72.39) (end 82.18 72.39) (width 0.25) (layer "F.Cu") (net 17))
 (segment (start 68.7316 81.779999) (end 72.889999 81.779999) (width 0.25) (layer "F.Cu") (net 17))
 (segment (start 73.66 82.55) (end 74.93 82.55) (width 0.25) (layer "F.Cu") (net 17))
 (segment (start 72.889999 81.779999) (end 73.66 82.55) (width 0.25) (layer "F.Cu") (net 17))
 (via (at 74.93 82.55) (size 0.8) (drill 0.4) (layers "F.Cu" "B.Cu") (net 17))
 (via (at 80.01 72.39) (size 0.8) (drill 0.4) (layers "F.Cu" "B.Cu") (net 17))
 (segment (start 78.74 81.28) (end 76.2 81.28) (width 0.25) (layer "B.Cu") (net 17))
 (segment (start 80.01 80.01) (end 78.74 81.28) (width 0.25) (layer "B.Cu") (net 17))
 (segment (start 76.2 81.28) (end 74.93 82.55) (width 0.25) (layer "B.Cu") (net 17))
 (segment (start 80.01 72.39) (end 80.01 80.01) (width 0.25) (layer "B.Cu") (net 17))
 (segment (start 68.7316 59.92) (end 71.35 59.92) (width 0.25) (layer "F.Cu") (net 3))
 (segment (start 72.39 60.96) (end 71.35 59.92) (width 0.25) (layer "F.Cu") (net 3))
 (segment (start 78.74 49.53) (end 82.18 49.53) (width 0.25) (layer "F.Cu") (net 3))
 (segment (start 73.66 60.96) (end 72.39 60.96) (width 0.25) (layer "F.Cu") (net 3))
 (via (at 78.74 49.53) (size 0.8) (drill 0.4) (layers "F.Cu" "B.Cu") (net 3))
 (via (at 73.66 60.96) (size 0.8) (drill 0.4) (layers "F.Cu" "B.Cu") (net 3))
 (segment (start 77.47 60.96) (end 73.66 60.96) (width 0.25) (layer "B.Cu") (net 3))
 (segment (start 78.74 59.69) (end 78.74 49.53) (width 0.25) (layer "B.Cu") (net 3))
 (segment (start 77.47 60.96) (end 78.74 59.69) (width 0.25) (layer "B.Cu") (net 3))
 (segment (start 68.7316 58.919999) (end 72.889999 58.919999) (width 0.25) (layer "F.Cu") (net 4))
 (segment (start 88 49.53) (end 86.73 48.26) (width 0.25) (layer "F.Cu") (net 4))
 (segment (start 72.889999 58.919999) (end 73.66 59.69) (width 0.25) (layer "F.Cu") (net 4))
 (segment (start 80.01 59.69) (end 77.47 59.69) (width 0.25) (layer "F.Cu") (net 4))
 (segment (start 86.73 48.26) (end 80.01 48.26) (width 0.25) (layer "F.Cu") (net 4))
 (via (at 80.01 59.69) (size 0.8) (drill 0.4) (layers "F.Cu" "B.Cu") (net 4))
 (via (at 77.47 59.69) (size 0.8) (drill 0.4) (layers "F.Cu" "B.Cu") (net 4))
 (via (at 80.01 48.26) (size 0.8) (drill 0.4) (layers "F.Cu" "B.Cu") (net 4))
 (via (at 73.66 59.69) (size 0.8) (drill 0.4) (layers "F.Cu" "B.Cu") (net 4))
 (segment (start 77.47 59.69) (end 73.66 59.69) (width 0.25) (layer "B.Cu") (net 4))
 (segment (start 80.01 48.26) (end 80.01 59.69) (width 0.25) (layer "B.Cu") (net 4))
 (segment (start 77.47 57.15) (end 77.47 58.42) (width 0.25) (layer "F.Cu") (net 5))
 (segment (start 68.7316 57.920001) (end 73.160001 57.920001) (width 0.5) (layer "F.Cu") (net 5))
 (segment (start 69.139791 34.33) (end 86.36 34.33) (width 0.5) (layer "F.Cu") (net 5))
 (segment (start 73.160001 57.920001) (end 73.66 58.42) (width 0.5) (layer "F.Cu") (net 5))
 (segment (start 76.2 57.15) (end 77.47 57.15) (width 0.5) (layer "F.Cu") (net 5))
 (segment (start 68.7316 46.490001) (end 72.889999 46.490001) (width 0.5) (layer "F.Cu") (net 5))
 (segment (start 76.2 45.72) (end 76.2 57.15) (width 0.5) (layer "F.Cu") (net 5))
 (segment (start 88 58.05) (end 88 54.61) (width 0.5) (layer "F.Cu") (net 5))
 (segment (start 87.63 58.42) (end 88 58.05) (width 0.5) (layer "F.Cu") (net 5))
 (segment (start 87.63 58.42) (end 77.47 58.42) (width 0.5) (layer "F.Cu") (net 5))
 (segment (start 72.889999 46.490001) (end 73.66 45.72) (width 0.5) (layer "F.Cu") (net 5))
 (via (at 86.36 34.33) (size 0.8) (drill 0.4) (layers "F.Cu" "B.Cu") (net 5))
 (via (at 87.63 58.42) (size 0.8) (drill 0.4) (layers "F.Cu" "B.Cu") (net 5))
 (via (at 73.66 45.72) (size 0.8) (drill 0.4) (layers "F.Cu" "B.Cu") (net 5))
 (via (at 77.47 58.42) (size 0.8) (drill 0.4) (layers "F.Cu" "B.Cu") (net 5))
 (via (at 73.66 58.42) (size 0.8) (drill 0.4) (layers "F.Cu" "B.Cu") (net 5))
 (via (at 76.2 45.72) (size 0.8) (drill 0.4) (layers "F.Cu" "B.Cu") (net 5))
 (via (at 77.47 57.15) (size 0.8) (drill 0.4) (layers "F.Cu" "B.Cu") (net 5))
 (segment (start 87.67 35.6) (end 88.9 36.83) (width 0.5) (layer "B.Cu") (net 5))
 (segment (start 73.66 58.42) (end 77.47 58.42) (width 0.5) (layer "B.Cu") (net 5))
 (segment (start 88.9 36.83) (end 88.9 57.15) (width 0.5) (layer "B.Cu") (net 5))
 (segment (start 73.66 45.72) (end 76.2 45.72) (width 0.5) (layer "B.Cu") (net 5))
 (segment (start 88.9 57.15) (end 87.63 58.42) (width 0.5) (layer "B.Cu") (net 5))
 (segment (start 87.63 35.6) (end 86.36 34.33) (width 0.5) (layer "B.Cu") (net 5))
 (segment (start 87.63 35.6) (end 87.67 35.6) (width 0.5) (layer "B.Cu") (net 5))
 (segment (start 80.01 63.5) (end 81.28 63.5) (width 0.25) (layer "F.Cu") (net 2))
 (segment (start 80.01 78.74) (end 87.63 78.74) (width 0.25) (layer "F.Cu") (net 2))
 (segment (start 77.47 76.2) (end 80.01 78.74) (width 0.25) (layer "F.Cu") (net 2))
 (segment (start 78.74 67.31) (end 78.74 71.12) (width 0.25) (layer "F.Cu") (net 2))
 (segment (start 78.74 71.12) (end 77.47 72.39) (width 0.25) (layer "F.Cu") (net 2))
 (segment (start 77.47 72.39) (end 77.47 76.2) (width 0.25) (layer "F.Cu") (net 2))
 (segment (start 88 79.11) (end 88 80.01) (width 0.25) (layer "F.Cu") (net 2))
 (segment (start 87.63 78.74) (end 88 79.11) (width 0.25) (layer "F.Cu") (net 2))
 (segment (start 81.28 63.5) (end 83.09 63.5) (width 0.25) (layer "F.Cu") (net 2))
 (via (at 81.28 63.5) (size 0.8) (drill 0.4) (layers "F.Cu" "B.Cu") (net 2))
 (via (at 78.74 67.31) (size 0.8) (drill 0.4) (layers "F.Cu" "B.Cu") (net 2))
 (segment (start 81.28 64.77) (end 78.74 67.31) (width 0.25) (layer "B.Cu") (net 2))
 (segment (start 81.28 63.5) (end 81.28 64.77) (width 0.25) (layer "B.Cu") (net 2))
 (segment (start 77.47 49.285305) (end 77.47 48.26) (width 0.25) (layer "F.Cu") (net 13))
 (segment (start 78.599695 50.415) (end 77.47 49.285305) (width 0.25) (layer "F.Cu") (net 13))
 (segment (start 86.345 50.415) (end 78.599695 50.415) (width 0.25) (layer "F.Cu") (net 13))
 (segment (start 68.7316 47.489999) (end 72.889999 47.489999) (width 0.25) (layer "F.Cu") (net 13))
 (segment (start 88 52.07) (end 86.345 50.415) (width 0.25) (layer "F.Cu") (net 13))
 (segment (start 72.889999 47.489999) (end 73.66 48.26) (width 0.25) (layer "F.Cu") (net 13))
 (via (at 77.47 48.26) (size 0.8) (drill 0.4) (layers "F.Cu" "B.Cu") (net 13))
 (via (at 73.66 48.26) (size 0.8) (drill 0.4) (layers "F.Cu" "B.Cu") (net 13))
 (segment (start 73.66 48.26) (end 77.47 48.26) (width 0.25) (layer "B.Cu") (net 13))
 (segment (start 68.7316 48.49) (end 71.35 48.49) (width 0.25) (layer "F.Cu") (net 12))
 (segment (start 77.47 52.07) (end 82.18 52.07) (width 0.25) (layer "F.Cu") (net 12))
 (segment (start 71.35 48.49) (end 73.66 50.8) (width 0.25) (layer "F.Cu") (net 12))
 (via (at 77.47 52.07) (size 0.8) (drill 0.4) (layers "F.Cu" "B.Cu") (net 12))
 (via (at 73.66 50.8) (size 0.8) (drill 0.4) (layers "F.Cu" "B.Cu") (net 12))
 (segment (start 77.47 52.07) (end 74.93 52.07) (width 0.25) (layer "B.Cu") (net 12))
 (segment (start 73.66 50.8) (end 74.93 52.07) (width 0.25) (layer "B.Cu") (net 12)))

